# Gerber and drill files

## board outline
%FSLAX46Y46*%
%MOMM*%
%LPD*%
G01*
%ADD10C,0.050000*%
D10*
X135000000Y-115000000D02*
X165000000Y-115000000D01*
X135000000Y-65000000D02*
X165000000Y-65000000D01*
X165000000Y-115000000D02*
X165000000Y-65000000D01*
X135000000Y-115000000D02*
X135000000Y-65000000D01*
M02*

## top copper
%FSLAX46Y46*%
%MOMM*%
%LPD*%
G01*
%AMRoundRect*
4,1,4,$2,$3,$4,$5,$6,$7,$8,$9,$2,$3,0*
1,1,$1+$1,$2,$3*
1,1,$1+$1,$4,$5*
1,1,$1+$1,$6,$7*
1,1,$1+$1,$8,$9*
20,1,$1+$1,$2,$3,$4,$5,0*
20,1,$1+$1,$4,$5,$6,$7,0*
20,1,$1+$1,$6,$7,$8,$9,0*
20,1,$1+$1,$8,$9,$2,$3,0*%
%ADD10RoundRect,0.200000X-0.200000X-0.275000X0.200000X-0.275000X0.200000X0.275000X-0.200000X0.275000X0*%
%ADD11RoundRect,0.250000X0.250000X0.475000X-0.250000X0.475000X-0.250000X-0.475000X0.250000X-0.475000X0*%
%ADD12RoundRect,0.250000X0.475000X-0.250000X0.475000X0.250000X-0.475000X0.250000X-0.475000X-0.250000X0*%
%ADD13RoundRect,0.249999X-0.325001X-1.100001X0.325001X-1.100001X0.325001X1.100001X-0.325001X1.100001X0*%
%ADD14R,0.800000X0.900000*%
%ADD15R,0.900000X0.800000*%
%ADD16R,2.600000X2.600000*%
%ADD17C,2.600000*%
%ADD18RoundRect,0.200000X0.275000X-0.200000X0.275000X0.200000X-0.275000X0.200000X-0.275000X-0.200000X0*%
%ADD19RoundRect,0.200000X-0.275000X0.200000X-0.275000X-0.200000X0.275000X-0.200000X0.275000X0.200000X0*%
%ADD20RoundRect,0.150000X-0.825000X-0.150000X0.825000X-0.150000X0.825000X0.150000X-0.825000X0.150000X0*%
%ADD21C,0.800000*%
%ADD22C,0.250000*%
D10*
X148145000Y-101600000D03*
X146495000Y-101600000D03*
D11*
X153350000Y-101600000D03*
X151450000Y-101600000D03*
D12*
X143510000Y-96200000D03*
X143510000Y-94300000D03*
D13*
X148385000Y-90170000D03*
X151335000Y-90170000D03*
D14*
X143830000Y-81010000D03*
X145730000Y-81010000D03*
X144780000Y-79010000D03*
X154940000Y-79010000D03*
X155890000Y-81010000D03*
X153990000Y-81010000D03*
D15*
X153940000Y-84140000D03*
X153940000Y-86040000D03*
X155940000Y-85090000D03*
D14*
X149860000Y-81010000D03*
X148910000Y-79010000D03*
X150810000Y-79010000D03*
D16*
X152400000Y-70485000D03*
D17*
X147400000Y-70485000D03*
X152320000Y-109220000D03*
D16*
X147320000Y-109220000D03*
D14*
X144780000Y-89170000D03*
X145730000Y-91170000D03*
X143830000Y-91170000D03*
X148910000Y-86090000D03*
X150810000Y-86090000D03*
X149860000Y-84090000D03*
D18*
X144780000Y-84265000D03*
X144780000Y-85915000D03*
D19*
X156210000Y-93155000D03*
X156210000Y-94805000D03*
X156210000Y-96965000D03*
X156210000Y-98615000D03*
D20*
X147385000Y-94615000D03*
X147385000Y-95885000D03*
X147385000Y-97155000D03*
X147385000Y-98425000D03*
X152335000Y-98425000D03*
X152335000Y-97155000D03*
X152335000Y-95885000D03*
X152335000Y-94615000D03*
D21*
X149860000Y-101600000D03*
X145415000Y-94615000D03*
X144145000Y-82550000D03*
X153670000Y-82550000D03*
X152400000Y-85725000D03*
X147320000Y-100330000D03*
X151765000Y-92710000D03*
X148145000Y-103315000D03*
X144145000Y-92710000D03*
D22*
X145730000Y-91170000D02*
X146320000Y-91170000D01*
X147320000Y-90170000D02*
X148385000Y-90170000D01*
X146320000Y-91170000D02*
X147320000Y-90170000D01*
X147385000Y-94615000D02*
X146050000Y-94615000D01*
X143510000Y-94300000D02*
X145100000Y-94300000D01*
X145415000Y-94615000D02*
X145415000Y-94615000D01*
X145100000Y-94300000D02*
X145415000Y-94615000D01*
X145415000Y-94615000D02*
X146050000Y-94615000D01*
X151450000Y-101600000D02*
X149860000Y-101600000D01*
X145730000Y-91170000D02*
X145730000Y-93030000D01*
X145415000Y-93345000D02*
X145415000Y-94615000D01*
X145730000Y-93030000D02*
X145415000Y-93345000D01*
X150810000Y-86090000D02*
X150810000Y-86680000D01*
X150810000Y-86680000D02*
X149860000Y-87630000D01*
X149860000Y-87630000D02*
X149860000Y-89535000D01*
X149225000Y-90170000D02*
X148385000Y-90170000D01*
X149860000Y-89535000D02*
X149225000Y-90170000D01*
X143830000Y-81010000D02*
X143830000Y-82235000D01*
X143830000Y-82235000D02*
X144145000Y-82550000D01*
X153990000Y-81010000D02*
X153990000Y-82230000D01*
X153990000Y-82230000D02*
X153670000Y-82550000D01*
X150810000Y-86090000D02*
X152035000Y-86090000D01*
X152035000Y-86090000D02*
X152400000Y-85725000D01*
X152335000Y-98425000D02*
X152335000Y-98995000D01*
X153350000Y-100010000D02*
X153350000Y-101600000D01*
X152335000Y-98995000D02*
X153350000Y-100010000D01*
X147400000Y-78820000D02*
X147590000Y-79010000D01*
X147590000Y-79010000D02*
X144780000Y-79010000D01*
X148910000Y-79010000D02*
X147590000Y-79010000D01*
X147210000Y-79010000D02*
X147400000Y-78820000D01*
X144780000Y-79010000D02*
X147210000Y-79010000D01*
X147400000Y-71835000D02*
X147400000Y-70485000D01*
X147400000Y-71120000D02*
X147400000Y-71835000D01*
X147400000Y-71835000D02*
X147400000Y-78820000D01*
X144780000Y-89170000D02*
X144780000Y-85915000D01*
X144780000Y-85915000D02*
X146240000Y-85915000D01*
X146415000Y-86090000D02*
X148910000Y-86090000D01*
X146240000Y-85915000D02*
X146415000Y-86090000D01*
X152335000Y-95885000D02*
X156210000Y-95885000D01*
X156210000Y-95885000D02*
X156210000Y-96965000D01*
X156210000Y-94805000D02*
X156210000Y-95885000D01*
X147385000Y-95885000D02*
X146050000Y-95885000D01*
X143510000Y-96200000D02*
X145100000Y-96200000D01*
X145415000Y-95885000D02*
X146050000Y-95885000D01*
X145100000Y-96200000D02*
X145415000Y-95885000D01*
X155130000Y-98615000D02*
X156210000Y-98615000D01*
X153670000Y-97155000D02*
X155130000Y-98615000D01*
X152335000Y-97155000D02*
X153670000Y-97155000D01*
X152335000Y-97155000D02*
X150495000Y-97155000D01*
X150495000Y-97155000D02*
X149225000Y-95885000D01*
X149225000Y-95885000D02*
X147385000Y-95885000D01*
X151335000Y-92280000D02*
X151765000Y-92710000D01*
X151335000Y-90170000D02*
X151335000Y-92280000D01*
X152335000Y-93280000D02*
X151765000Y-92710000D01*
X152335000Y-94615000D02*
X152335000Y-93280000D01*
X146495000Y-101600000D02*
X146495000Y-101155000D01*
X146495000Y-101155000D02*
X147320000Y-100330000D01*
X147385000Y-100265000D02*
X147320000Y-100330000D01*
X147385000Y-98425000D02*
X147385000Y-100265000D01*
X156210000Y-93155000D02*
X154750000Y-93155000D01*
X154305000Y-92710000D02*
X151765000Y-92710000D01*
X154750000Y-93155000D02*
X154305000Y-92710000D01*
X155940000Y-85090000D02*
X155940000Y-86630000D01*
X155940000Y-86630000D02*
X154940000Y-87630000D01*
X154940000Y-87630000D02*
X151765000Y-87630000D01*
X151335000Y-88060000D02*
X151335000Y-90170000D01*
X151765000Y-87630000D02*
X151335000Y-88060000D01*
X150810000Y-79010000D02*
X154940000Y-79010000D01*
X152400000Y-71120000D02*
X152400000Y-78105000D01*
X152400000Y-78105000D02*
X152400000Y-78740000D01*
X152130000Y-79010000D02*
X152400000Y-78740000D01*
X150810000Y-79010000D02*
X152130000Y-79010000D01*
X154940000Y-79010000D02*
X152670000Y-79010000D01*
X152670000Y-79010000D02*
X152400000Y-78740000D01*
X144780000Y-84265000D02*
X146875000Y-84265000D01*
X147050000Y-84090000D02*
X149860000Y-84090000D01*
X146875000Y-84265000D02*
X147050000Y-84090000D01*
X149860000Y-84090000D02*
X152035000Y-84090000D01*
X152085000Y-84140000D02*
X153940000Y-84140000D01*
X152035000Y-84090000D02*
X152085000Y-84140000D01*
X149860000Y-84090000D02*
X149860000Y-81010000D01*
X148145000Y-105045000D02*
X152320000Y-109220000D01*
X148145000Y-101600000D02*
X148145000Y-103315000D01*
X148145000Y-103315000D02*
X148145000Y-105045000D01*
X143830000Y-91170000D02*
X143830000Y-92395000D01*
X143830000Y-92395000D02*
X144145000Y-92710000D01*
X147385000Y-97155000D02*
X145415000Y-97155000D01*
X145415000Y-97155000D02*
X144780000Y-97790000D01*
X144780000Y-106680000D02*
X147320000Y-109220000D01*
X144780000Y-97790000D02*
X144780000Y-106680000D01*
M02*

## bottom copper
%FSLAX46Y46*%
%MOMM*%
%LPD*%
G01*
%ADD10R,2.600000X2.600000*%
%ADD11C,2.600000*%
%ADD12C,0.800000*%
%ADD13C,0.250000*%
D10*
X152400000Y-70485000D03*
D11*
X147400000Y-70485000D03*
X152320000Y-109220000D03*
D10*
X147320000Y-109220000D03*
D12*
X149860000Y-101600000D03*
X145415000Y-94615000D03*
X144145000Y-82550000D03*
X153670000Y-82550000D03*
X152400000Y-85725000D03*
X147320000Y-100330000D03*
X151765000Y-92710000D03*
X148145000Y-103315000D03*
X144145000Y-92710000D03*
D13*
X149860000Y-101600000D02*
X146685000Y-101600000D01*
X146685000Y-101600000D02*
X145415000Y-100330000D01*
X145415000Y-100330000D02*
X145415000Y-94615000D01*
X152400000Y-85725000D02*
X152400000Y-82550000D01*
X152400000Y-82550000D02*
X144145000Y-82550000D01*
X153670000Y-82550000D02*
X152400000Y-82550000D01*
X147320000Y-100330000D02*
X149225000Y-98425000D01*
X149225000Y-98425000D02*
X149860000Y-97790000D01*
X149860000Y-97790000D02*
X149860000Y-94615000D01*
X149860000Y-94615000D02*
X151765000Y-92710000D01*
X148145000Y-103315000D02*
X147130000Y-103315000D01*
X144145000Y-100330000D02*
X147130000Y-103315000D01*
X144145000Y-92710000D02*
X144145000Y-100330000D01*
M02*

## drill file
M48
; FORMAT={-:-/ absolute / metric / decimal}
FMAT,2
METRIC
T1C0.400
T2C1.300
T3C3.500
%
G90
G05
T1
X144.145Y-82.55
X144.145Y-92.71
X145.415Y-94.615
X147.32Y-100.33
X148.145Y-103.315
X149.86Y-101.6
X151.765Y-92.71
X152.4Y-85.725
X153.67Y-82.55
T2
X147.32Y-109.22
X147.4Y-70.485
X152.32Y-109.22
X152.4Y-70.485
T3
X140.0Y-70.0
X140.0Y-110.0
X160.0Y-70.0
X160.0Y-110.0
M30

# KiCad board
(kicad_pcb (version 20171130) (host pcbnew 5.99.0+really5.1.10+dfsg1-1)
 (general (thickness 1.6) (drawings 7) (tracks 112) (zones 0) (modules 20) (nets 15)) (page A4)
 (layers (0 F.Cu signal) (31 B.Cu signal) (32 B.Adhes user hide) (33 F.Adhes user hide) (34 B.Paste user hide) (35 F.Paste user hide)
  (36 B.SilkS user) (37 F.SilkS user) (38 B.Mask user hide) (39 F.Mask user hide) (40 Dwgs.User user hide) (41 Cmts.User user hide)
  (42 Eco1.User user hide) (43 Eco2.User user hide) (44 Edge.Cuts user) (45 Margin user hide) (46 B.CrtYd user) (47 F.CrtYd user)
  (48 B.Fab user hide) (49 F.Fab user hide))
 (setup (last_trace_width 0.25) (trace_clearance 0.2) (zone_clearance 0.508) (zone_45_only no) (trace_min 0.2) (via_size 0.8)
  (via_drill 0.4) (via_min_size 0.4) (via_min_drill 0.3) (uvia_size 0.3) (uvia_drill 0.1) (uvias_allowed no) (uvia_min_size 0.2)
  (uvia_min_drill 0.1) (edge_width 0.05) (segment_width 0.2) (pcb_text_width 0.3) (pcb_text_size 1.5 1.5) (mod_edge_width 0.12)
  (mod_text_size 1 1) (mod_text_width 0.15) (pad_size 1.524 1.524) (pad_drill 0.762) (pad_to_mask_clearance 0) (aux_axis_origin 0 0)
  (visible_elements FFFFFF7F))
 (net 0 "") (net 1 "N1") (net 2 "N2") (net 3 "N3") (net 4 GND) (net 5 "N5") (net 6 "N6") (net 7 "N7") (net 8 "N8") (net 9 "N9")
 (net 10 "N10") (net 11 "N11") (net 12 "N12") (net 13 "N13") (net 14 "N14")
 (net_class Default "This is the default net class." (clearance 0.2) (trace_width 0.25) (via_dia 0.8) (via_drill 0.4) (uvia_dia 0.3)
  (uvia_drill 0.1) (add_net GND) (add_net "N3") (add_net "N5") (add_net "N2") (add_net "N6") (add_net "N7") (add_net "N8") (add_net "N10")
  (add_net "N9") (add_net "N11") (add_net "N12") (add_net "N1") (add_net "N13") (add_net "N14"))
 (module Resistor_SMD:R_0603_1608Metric (layer F.Cu) (at 147.32 101.6)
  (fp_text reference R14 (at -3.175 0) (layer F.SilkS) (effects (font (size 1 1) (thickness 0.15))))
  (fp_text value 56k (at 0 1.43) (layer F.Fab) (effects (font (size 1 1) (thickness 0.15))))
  (pad 2 smd roundrect (at 0.825 0) (size 0.8 0.95) (layers F.Cu F.Paste F.Mask) (roundrect_rratio 0.25) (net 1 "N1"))
  (pad 1 smd roundrect (at -0.825 0) (size 0.8 0.95) (layers F.Cu F.Paste F.Mask) (roundrect_rratio 0.25) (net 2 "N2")))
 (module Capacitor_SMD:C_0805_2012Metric (layer F.Cu) (at 152.4 101.6 180)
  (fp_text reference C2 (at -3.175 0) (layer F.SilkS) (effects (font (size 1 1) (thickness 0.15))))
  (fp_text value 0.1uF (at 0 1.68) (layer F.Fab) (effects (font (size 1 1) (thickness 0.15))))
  (pad 1 smd roundrect (at -0.95 0 180) (size 1 1.45) (layers F.Cu F.Paste F.Mask) (roundrect_rratio 0.25) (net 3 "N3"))
  (pad 2 smd roundrect (at 0.95 0 180) (size 1 1.45) (layers F.Cu F.Paste F.Mask) (roundrect_rratio 0.25) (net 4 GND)))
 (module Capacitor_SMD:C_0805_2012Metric (layer F.Cu) (at 143.51 95.25 90)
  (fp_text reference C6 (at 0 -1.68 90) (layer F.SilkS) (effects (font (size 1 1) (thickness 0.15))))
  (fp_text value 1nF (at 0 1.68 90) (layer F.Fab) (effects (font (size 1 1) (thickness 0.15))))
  (pad 1 smd roundrect (at -0.95 0 90) (size 1 1.45) (layers F.Cu F.Paste F.Mask) (roundrect_rratio 0.25) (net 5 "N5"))
  (pad 2 smd roundrect (at 0.95 0 90) (size 1 1.45) (layers F.Cu F.Paste F.Mask) (roundrect_rratio 0.25) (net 4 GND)))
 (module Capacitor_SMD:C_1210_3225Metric (layer F.Cu) (at 149.86 90.17)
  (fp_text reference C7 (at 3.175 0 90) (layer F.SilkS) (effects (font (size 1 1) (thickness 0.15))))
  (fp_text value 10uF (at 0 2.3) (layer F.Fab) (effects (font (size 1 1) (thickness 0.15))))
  (pad 1 smd roundrect (at -1.475 0) (size 1.15 2.7) (layers F.Cu F.Paste F.Mask) (roundrect_rratio 0.2173904347826087) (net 4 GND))
  (pad 2 smd roundrect (at 1.475 0) (size 1.15 2.7) (layers F.Cu F.Paste F.Mask) (roundrect_rratio 0.2173904347826087) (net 2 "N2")))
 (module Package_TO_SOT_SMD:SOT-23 (layer F.Cu) (at 144.78 80.01 90)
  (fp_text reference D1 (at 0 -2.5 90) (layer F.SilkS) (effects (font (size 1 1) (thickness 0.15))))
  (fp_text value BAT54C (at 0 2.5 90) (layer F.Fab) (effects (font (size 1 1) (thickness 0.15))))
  (pad 1 smd rect (at -1 -0.95 90) (size 0.9 0.8) (layers F.Cu F.Paste F.Mask) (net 4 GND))
  (pad 2 smd rect (at -1 0.95 90) (size 0.9 0.8) (layers F.Cu F.Paste F.Mask) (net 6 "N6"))
  (pad 3 smd rect (at 1 0 90) (size 0.9 0.8) (layers F.Cu F.Paste F.Mask) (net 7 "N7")))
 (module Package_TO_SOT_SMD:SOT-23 (layer F.Cu) (at 154.94 80.01 90)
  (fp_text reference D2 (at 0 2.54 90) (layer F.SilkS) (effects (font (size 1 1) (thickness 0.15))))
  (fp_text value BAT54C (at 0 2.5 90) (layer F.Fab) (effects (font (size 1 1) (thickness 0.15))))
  (pad 3 smd rect (at 1 0 90) (size 0.9 0.8) (layers F.Cu F.Paste F.Mask) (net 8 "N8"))
  (pad 2 smd rect (at -1 0.95 90) (size 0.9 0.8) (layers F.Cu F.Paste F.Mask) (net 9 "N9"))
  (pad 1 smd rect (at -1 -0.95 90) (size 0.9 0.8) (layers F.Cu F.Paste F.Mask) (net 4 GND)))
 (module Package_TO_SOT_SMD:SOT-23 (layer F.Cu) (at 154.94 85.09)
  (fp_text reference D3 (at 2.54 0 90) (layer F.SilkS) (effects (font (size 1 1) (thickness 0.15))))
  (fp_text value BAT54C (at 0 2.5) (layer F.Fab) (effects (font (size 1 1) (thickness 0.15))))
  (pad 1 smd rect (at -1 -0.95) (size 0.9 0.8) (layers F.Cu F.Paste F.Mask) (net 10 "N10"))
  (pad 2 smd rect (at -1 0.95) (size 0.9 0.8) (layers F.Cu F.Paste F.Mask) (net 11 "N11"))
  (pad 3 smd rect (at 1 0) (size 0.9 0.8) (layers F.Cu F.Paste F.Mask) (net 2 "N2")))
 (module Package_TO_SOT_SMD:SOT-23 (layer F.Cu) (at 149.86 80.01 270)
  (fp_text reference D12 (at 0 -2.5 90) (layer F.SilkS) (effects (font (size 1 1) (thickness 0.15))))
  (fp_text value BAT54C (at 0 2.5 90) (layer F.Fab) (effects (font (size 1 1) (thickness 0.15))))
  (pad 3 smd rect (at 1 0 270) (size 0.9 0.8) (layers F.Cu F.Paste F.Mask) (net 10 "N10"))
  (pad 2 smd rect (at -1 0.95 270) (size 0.9 0.8) (layers F.Cu F.Paste F.Mask) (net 7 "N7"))
  (pad 1 smd rect (at -1 -0.95 270) (size 0.9 0.8) (layers F.Cu F.Paste F.Mask) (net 8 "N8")))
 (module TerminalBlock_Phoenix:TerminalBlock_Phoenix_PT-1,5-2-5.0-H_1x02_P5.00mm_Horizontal (layer F.Cu) (at 152.4 70.485 180)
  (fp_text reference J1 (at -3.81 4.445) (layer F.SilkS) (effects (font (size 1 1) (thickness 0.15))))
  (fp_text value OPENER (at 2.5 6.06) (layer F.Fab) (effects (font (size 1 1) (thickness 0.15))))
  (pad 1 thru_hole rect (at 0 0 180) (size 2.6 2.6) (drill 1.3) (layers *.Cu *.Mask) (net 8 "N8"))
  (pad 2 thru_hole circle (at 5 0 180) (size 2.6 2.6) (drill 1.3) (layers *.Cu *.Mask) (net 7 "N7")))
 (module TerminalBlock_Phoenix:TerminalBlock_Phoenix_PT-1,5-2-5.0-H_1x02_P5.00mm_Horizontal (layer F.Cu) (at 147.32 109.22)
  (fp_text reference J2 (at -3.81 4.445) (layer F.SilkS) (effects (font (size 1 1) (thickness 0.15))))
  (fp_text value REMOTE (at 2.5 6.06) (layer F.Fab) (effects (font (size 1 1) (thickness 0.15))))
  (pad 2 thru_hole circle (at 5 0) (size 2.6 2.6) (drill 1.3) (layers *.Cu *.Mask) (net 1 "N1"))
  (pad 1 thru_hole rect (at 0 0) (size 2.6 2.6) (drill 1.3) (layers *.Cu *.Mask) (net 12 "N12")))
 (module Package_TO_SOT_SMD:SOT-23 (layer F.Cu) (at 144.78 90.17 90)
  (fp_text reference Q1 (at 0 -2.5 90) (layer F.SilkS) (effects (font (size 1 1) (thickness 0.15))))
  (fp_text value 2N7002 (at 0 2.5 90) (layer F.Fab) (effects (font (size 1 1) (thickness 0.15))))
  (pad 3 smd rect (at 1 0 90) (size 0.9 0.8) (layers F.Cu F.Paste F.Mask) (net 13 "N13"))
  (pad 2 smd rect (at -1 0.95 90) (size 0.9 0.8) (layers F.Cu F.Paste F.Mask) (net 4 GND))
  (pad 1 smd rect (at -1 -0.95 90) (size 0.9 0.8) (layers F.Cu F.Paste F.Mask) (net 1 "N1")))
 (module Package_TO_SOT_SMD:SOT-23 (layer F.Cu) (at 149.86 85.09 90)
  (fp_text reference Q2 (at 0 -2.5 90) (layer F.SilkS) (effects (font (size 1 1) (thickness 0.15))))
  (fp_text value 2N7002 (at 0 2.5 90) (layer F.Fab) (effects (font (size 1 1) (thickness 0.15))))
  (pad 1 smd rect (at -1 -0.95 90) (size 0.9 0.8) (layers F.Cu F.Paste F.Mask) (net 13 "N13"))
  (pad 2 smd rect (at -1 0.95 90) (size 0.9 0.8) (layers F.Cu F.Paste F.Mask) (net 4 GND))
  (pad 3 smd rect (at 1 0 90) (size 0.9 0.8) (layers F.Cu F.Paste F.Mask) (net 10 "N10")))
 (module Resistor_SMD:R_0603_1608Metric (layer F.Cu) (at 144.78 85.09 90)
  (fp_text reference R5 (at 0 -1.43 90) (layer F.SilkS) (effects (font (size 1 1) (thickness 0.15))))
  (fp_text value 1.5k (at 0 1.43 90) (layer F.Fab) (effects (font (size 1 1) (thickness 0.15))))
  (pad 2 smd roundrect (at 0.825 0 90) (size 0.8 0.95) (layers F.Cu F.Paste F.Mask) (roundrect_rratio 0.25) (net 10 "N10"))
  (pad 1 smd roundrect (at -0.825 0 90) (size 0.8 0.95) (layers F.Cu F.Paste F.Mask) (roundrect_rratio 0.25) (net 13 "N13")))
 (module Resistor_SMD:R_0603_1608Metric (layer F.Cu) (at 156.21 93.98 270)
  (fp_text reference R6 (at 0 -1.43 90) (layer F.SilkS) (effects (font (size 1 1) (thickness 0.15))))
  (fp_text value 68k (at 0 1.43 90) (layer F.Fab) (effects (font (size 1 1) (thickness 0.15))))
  (pad 1 smd roundrect (at -0.825 0 270) (size 0.8 0.95) (layers F.Cu F.Paste F.Mask) (roundrect_rratio 0.25) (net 2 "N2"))
  (pad 2 smd roundrect (at 0.825 0 270) (size 0.8 0.95) (layers F.Cu F.Paste F.Mask) (roundrect_rratio 0.25) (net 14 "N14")))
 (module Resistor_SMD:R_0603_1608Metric (layer F.Cu) (at 156.21 97.79 270)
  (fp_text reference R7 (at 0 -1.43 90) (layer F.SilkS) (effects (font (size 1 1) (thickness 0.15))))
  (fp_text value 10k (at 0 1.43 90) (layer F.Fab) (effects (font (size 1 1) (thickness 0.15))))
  (pad 1 smd roundrect (at -0.825 0 270) (size 0.8 0.95) (layers F.Cu F.Paste F.Mask) (roundrect_rratio 0.25) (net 14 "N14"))
  (pad 2 smd roundrect (at 0.825 0 270) (size 0.8 0.95) (layers F.Cu F.Paste F.Mask) (roundrect_rratio 0.25) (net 5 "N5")))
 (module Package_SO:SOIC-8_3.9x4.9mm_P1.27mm (layer F.Cu) (at 149.86 96.52)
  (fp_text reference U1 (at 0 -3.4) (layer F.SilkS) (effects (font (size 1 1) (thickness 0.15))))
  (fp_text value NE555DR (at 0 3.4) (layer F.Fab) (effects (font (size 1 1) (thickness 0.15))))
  (pad 1 smd roundrect (at -2.475 -1.905) (size 1.95 0.6) (layers F.Cu F.Paste F.Mask) (roundrect_rratio 0.25) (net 4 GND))
  (pad 2 smd roundrect (at -2.475 -0.635) (size 1.95 0.6) (layers F.Cu F.Paste F.Mask) (roundrect_rratio 0.25) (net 5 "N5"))
  (pad 3 smd roundrect (at -2.475 0.635) (size 1.95 0.6) (layers F.Cu F.Paste F.Mask) (roundrect_rratio 0.25) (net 12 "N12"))
  (pad 4 smd roundrect (at -2.475 1.905) (size 1.95 0.6) (layers F.Cu F.Paste F.Mask) (roundrect_rratio 0.25) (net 2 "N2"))
  (pad 5 smd roundrect (at 2.475 1.905) (size 1.95 0.6) (layers F.Cu F.Paste F.Mask) (roundrect_rratio 0.25) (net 3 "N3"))
  (pad 6 smd roundrect (at 2.475 0.635) (size 1.95 0.6) (layers F.Cu F.Paste F.Mask) (roundrect_rratio 0.25) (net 5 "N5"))
  (pad 7 smd roundrect (at 2.475 -0.635) (size 1.95 0.6) (layers F.Cu F.Paste F.Mask) (roundrect_rratio 0.25) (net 14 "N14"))
  (pad 8 smd roundrect (at 2.475 -1.905) (size 1.95 0.6) (layers F.Cu F.Paste F.Mask) (roundrect_rratio 0.25) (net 2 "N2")))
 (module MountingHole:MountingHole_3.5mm (layer F.Cu) (at 160 70)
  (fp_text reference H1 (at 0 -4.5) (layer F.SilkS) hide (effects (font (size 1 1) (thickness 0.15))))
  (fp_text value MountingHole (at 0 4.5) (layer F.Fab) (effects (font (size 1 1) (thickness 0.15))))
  (pad 1 np_thru_hole circle (at 0 0) (size 3.5 3.5) (drill 3.5) (layers *.Cu *.Mask)))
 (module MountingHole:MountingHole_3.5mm (layer F.Cu) (at 140 70)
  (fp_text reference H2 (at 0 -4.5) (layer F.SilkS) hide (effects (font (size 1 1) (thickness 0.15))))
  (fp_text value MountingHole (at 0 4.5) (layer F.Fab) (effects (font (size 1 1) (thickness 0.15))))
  (pad 1 np_thru_hole circle (at 0 0) (size 3.5 3.5) (drill 3.5) (layers *.Cu *.Mask)))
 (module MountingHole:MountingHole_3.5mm (layer F.Cu) (at 140 110)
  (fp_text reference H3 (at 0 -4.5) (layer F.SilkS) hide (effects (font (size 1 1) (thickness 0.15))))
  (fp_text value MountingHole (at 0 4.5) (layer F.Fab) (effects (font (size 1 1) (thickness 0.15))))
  (pad 1 np_thru_hole circle (at 0 0) (size 3.5 3.5) (drill 3.5) (layers *.Cu *.Mask)))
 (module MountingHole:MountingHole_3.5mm (layer F.Cu) (at 160 110)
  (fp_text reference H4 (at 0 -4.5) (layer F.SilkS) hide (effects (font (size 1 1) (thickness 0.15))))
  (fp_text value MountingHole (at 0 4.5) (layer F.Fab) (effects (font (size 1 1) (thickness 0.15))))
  (pad 1 np_thru_hole circle (at 0 0) (size 3.5 3.5) (drill 3.5) (layers *.Cu *.Mask)))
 (gr_line (start 135 115) (end 165 115) (layer Edge.Cuts) (width 0.05))
 (gr_line (start 135 65) (end 165 65) (layer Edge.Cuts) (width 0.05))
 (gr_line (start 165 115) (end 165 65) (layer Edge.Cuts) (width 0.05))
 (gr_line (start 135 115) (end 135 65) (layer Edge.Cuts) (width 0.05))
 (segment (start 145.73 91.17) (end 146.32 91.17) (width 0.25) (layer F.Cu) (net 4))
 (segment (start 147.32 90.17) (end 148.385 90.17) (width 0.25) (layer F.Cu) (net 4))
 (segment (start 146.32 91.17) (end 147.32 90.17) (width 0.25) (layer F.Cu) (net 4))
 (segment (start 147.385 94.615) (end 146.05 94.615) (width 0.25) (layer F.Cu) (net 4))
 (segment (start 143.51 94.3) (end 145.1 94.3) (width 0.25) (layer F.Cu) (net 4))
 (segment (start 145.415 94.615) (end 145.415 94.615) (width 0.25) (layer F.Cu) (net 4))
 (segment (start 145.1 94.3) (end 145.415 94.615) (width 0.25) (layer F.Cu) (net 4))
 (segment (start 145.415 94.615) (end 146.05 94.615) (width 0.25) (layer F.Cu) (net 4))
 (segment (start 151.45 101.6) (end 149.86 101.6) (width 0.25) (layer F.Cu) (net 4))
 (via (at 149.86 101.6) (size 0.8) (drill 0.4) (layers F.Cu B.Cu) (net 4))
 (segment (start 149.86 101.6) (end 146.685 101.6) (width 0.25) (layer B.Cu) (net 4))
 (segment (start 146.685 101.6) (end 145.415 100.33) (width 0.25) (layer B.Cu) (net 4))
 (segment (start 145.415 100.33) (end 145.415 94.615) (width 0.25) (layer B.Cu) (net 4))
 (via (at 145.415 94.615) (size 0.8) (drill 0.4) (layers F.Cu B.Cu) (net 4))
 (segment (start 145.73 91.17) (end 145.73 93.03) (width 0.25) (layer F.Cu) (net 4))
 (segment (start 145.415 93.345) (end 145.415 94.615) (width 0.25) (layer F.Cu) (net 4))
 (segment (start 145.73 93.03) (end 145.415 93.345) (width 0.25) (layer F.Cu) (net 4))
 (segment (start 150.81 86.09) (end 150.81 86.68) (width 0.25) (layer F.Cu) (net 4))
 (segment (start 150.81 86.68) (end 149.86 87.63) (width 0.25) (layer F.Cu) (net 4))
 (segment (start 149.86 87.63) (end 149.86 89.535) (width 0.25) (layer F.Cu) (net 4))
 (segment (start 149.225 90.17) (end 148.385 90.17) (width 0.25) (layer F.Cu) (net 4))
 (segment (start 149.86 89.535) (end 149.225 90.17) (width 0.25) (layer F.Cu) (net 4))
 (segment (start 143.83 81.01) (end 143.83 82.235) (width 0.25) (layer F.Cu) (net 4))
 (segment (start 143.83 82.235) (end 144.145 82.55) (width 0.25) (layer F.Cu) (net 4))
 (via (at 144.145 82.55) (size 0.8) (drill 0.4) (layers F.Cu B.Cu) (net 4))
 (segment (start 153.99 81.01) (end 153.99 82.23) (width 0.25) (layer F.Cu) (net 4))
 (via (at 153.67 82.55) (size 0.8) (drill 0.4) (layers F.Cu B.Cu) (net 4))
 (segment (start 153.99 82.23) (end 153.67 82.55) (width 0.25) (layer F.Cu) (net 4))
 (segment (start 150.81 86.09) (end 152.035 86.09) (width 0.25) (layer F.Cu) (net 4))
 (via (at 152.4 85.725) (size 0.8) (drill 0.4) (layers F.Cu B.Cu) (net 4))
 (segment (start 152.035 86.09) (end 152.4 85.725) (width 0.25) (layer F.Cu) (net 4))
 (segment (start 152.4 85.725) (end 152.4 82.55) (width 0.25) (layer B.Cu) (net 4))
 (segment (start 152.4 82.55) (end 144.145 82.55) (width 0.25) (layer B.Cu) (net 4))
 (segment (start 153.67 82.55) (end 152.4 82.55) (width 0.25) (layer B.Cu) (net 4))
 (segment (start 152.335 98.425) (end 152.335 98.995) (width 0.25) (layer F.Cu) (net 3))
 (segment (start 153.35 100.01) (end 153.35 101.6) (width 0.25) (layer F.Cu) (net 3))
 (segment (start 152.335 98.995) (end 153.35 100.01) (width 0.25) (layer F.Cu) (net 3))
 (segment (start 147.4 78.82) (end 147.59 79.01) (width 0.25) (layer F.Cu) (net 7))
 (segment (start 147.59 79.01) (end 144.78 79.01) (width 0.25) (layer F.Cu) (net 7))
 (segment (start 148.91 79.01) (end 147.59 79.01) (width 0.25) (layer F.Cu) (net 7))
 (segment (start 147.21 79.01) (end 147.4 78.82) (width 0.25) (layer F.Cu) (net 7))
 (segment (start 144.78 79.01) (end 147.21 79.01) (width 0.25) (layer F.Cu) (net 7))
 (segment (start 147.4 71.835) (end 147.4 70.485) (width 0.25) (layer F.Cu) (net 7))
 (segment (start 147.4 71.12) (end 147.4 71.835) (width 0.25) (layer F.Cu) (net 7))
 (segment (start 147.4 71.835) (end 147.4 78.82) (width 0.25) (layer F.Cu) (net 7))
 (segment (start 144.78 89.17) (end 144.78 85.915) (width 0.25) (layer F.Cu) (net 13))
 (segment (start 144.78 85.915) (end 146.24 85.915) (width 0.25) (layer F.Cu) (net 13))
 (segment (start 146.415 86.09) (end 148.91 86.09) (width 0.25) (layer F.Cu) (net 13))
 (segment (start 146.24 85.915) (end 146.415 86.09) (width 0.25) (layer F.Cu) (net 13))
 (segment (start 152.335 95.885) (end 156.21 95.885) (width 0.25) (layer F.Cu) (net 14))
 (segment (start 156.21 95.885) (end 156.21 96.965) (width 0.25) (layer F.Cu) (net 14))
 (segment (start 156.21 94.805) (end 156.21 95.885) (width 0.25) (layer F.Cu) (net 14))
 (segment (start 147.385 95.885) (end 146.05 95.885) (width 0.25) (layer F.Cu) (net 5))
 (segment (start 143.51 96.2) (end 145.1 96.2) (width 0.25) (layer F.Cu) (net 5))
 (segment (start 145.415 95.885) (end 146.05 95.885) (width 0.25) (layer F.Cu) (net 5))
 (segment (start 145.1 96.2) (end 145.415 95.885) (width 0.25) (layer F.Cu) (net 5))
 (segment (start 155.13 98.615) (end 156.21 98.615) (width 0.25) (layer F.Cu) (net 5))
 (segment (start 153.67 97.155) (end 155.13 98.615) (width 0.25) (layer F.Cu) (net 5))
 (segment (start 152.335 97.155) (end 153.67 97.155) (width 0.25) (layer F.Cu) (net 5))
 (segment (start 152.335 97.155) (end 150.495 97.155) (width 0.25) (layer F.Cu) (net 5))
 (segment (start 150.495 97.155) (end 149.225 95.885) (width 0.25) (layer F.Cu) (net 5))
 (segment (start 149.225 95.885) (end 147.385 95.885) (width 0.25) (layer F.Cu) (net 5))
 (segment (start 151.335 92.28) (end 151.765 92.71) (width 0.25) (layer F.Cu) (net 2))
 (segment (start 151.335 90.17) (end 151.335 92.28) (width 0.25) (layer F.Cu) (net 2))
 (segment (start 152.335 93.28) (end 151.765 92.71) (width 0.25) (layer F.Cu) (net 2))
 (segment (start 152.335 94.615) (end 152.335 93.28) (width 0.25) (layer F.Cu) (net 2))
 (segment (start 146.495 101.6) (end 146.495 101.155) (width 0.25) (layer F.Cu) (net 2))
 (segment (start 146.495 101.155) (end 147.32 100.33) (width 0.25) (layer F.Cu) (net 2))
 (via (at 147.32 100.33) (size 0.8) (drill 0.4) (layers F.Cu B.Cu) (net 2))
 (segment (start 147.385 100.265) (end 147.32 100.33) (width 0.25) (layer F.Cu) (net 2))
 (segment (start 147.385 98.425) (end 147.385 100.265) (width 0.25) (layer F.Cu) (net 2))
 (segment (start 147.32 100.33) (end 149.225 98.425) (width 0.25) (layer B.Cu) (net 2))
 (segment (start 149.225 98.425) (end 149.86 97.79) (width 0.25) (layer B.Cu) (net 2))
 (segment (start 149.86 97.79) (end 149.86 94.615) (width 0.25) (layer B.Cu) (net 2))
 (segment (start 149.86 94.615) (end 151.765 92.71) (width 0.25) (layer B.Cu) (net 2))
 (via (at 151.765 92.71) (size 0.8) (drill 0.4) (layers F.Cu B.Cu) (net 2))
 (segment (start 156.21 93.155) (end 154.75 93.155) (width 0.25) (layer F.Cu) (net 2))
 (segment (start 154.305 92.71) (end 151.765 92.71) (width 0.25) (layer F.Cu) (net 2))
 (segment (start 154.75 93.155) (end 154.305 92.71) (width 0.25) (layer F.Cu) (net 2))
 (segment (start 155.94 85.09) (end 155.94 86.63) (width 0.25) (layer F.Cu) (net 2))
 (segment (start 155.94 86.63) (end 154.94 87.63) (width 0.25) (layer F.Cu) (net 2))
 (segment (start 154.94 87.63) (end 151.765 87.63) (width 0.25) (layer F.Cu) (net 2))
 (segment (start 151.335 88.06) (end 151.335 90.17) (width 0.25) (layer F.Cu) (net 2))
 (segment (start 151.765 87.63) (end 151.335 88.06) (width 0.25) (layer F.Cu) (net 2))
 (segment (start 150.81 79.01) (end 154.94 79.01) (width 0.25) (layer F.Cu) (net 8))
 (segment (start 152.4 71.12) (end 152.4 78.105) (width 0.25) (layer F.Cu) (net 8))
 (segment (start 152.4 78.105) (end 152.4 78.74) (width 0.25) (layer F.Cu) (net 8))
 (segment (start 152.13 79.01) (end 152.4 78.74) (width 0.25) (layer F.Cu) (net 8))
 (segment (start 150.81 79.01) (end 152.13 79.01) (width 0.25) (layer F.Cu) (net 8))
 (segment (start 154.94 79.01) (end 152.67 79.01) (width 0.25) (layer F.Cu) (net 8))
 (segment (start 152.67 79.01) (end 152.4 78.74) (width 0.25) (layer F.Cu) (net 8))
 (segment (start 144.78 84.265) (end 146.875 84.265) (width 0.25) (layer F.Cu) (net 10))
 (segment (start 147.05 84.09) (end 149.86 84.09) (width 0.25) (layer F.Cu) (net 10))
 (segment (start 146.875 84.265) (end 147.05 84.09) (width 0.25) (layer F.Cu) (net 10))
 (segment (start 149.86 84.09) (end 152.035 84.09) (width 0.25) (layer F.Cu) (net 10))
 (segment (start 152.085 84.14) (end 153.94 84.14) (width 0.25) (layer F.Cu) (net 10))
 (segment (start 152.035 84.09) (end 152.085 84.14) (width 0.25) (layer F.Cu) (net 10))
 (segment (start 149.86 84.09) (end 149.86 81.01) (width 0.25) (layer F.Cu) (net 10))
 (segment (start 148.145 105.045) (end 152.32 109.22) (width 0.25) (layer F.Cu) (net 1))
 (segment (start 148.145 101.6) (end 148.145 103.315) (width 0.25) (layer F.Cu) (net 1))
 (segment (start 148.145 103.315) (end 148.145 105.045) (width 0.25) (layer F.Cu) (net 1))
 (via (at 148.145 103.315) (size 0.8) (drill 0.4) (layers F.Cu B.Cu) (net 1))
 (segment (start 148.145 103.315) (end 147.13 103.315) (width 0.25) (layer B.Cu) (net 1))
 (segment (start 143.83 91.17) (end 143.83 92.395) (width 0.25) (layer F.Cu) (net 1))
 (segment (start 143.83 92.395) (end 144.145 92.71) (width 0.25) (layer F.Cu) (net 1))
 (via (at 144.145 92.71) (size 0.8) (drill 0.4) (layers F.Cu B.Cu) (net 1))
 (segment (start 144.145 100.33) (end 147.13 103.315) (width 0.25) (layer B.Cu) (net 1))
 (segment (start 144.145 92.71) (end 144.145 100.33) (width 0.25) (layer B.Cu) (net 1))
 (segment (start 147.385 97.155) (end 145.415 97.155) (width 0.25) (layer F.Cu) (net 12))
 (segment (start 145.415 97.155) (end 144.78 97.79) (width 0.25) (layer F.Cu) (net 12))
 (segment (start 144.78 106.68) (end 147.32 109.22) (width 0.25) (layer F.Cu) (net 12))
 (segment (start 144.78 97.79) (end 144.78 106.68) (width 0.25) (layer F.Cu) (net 12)))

